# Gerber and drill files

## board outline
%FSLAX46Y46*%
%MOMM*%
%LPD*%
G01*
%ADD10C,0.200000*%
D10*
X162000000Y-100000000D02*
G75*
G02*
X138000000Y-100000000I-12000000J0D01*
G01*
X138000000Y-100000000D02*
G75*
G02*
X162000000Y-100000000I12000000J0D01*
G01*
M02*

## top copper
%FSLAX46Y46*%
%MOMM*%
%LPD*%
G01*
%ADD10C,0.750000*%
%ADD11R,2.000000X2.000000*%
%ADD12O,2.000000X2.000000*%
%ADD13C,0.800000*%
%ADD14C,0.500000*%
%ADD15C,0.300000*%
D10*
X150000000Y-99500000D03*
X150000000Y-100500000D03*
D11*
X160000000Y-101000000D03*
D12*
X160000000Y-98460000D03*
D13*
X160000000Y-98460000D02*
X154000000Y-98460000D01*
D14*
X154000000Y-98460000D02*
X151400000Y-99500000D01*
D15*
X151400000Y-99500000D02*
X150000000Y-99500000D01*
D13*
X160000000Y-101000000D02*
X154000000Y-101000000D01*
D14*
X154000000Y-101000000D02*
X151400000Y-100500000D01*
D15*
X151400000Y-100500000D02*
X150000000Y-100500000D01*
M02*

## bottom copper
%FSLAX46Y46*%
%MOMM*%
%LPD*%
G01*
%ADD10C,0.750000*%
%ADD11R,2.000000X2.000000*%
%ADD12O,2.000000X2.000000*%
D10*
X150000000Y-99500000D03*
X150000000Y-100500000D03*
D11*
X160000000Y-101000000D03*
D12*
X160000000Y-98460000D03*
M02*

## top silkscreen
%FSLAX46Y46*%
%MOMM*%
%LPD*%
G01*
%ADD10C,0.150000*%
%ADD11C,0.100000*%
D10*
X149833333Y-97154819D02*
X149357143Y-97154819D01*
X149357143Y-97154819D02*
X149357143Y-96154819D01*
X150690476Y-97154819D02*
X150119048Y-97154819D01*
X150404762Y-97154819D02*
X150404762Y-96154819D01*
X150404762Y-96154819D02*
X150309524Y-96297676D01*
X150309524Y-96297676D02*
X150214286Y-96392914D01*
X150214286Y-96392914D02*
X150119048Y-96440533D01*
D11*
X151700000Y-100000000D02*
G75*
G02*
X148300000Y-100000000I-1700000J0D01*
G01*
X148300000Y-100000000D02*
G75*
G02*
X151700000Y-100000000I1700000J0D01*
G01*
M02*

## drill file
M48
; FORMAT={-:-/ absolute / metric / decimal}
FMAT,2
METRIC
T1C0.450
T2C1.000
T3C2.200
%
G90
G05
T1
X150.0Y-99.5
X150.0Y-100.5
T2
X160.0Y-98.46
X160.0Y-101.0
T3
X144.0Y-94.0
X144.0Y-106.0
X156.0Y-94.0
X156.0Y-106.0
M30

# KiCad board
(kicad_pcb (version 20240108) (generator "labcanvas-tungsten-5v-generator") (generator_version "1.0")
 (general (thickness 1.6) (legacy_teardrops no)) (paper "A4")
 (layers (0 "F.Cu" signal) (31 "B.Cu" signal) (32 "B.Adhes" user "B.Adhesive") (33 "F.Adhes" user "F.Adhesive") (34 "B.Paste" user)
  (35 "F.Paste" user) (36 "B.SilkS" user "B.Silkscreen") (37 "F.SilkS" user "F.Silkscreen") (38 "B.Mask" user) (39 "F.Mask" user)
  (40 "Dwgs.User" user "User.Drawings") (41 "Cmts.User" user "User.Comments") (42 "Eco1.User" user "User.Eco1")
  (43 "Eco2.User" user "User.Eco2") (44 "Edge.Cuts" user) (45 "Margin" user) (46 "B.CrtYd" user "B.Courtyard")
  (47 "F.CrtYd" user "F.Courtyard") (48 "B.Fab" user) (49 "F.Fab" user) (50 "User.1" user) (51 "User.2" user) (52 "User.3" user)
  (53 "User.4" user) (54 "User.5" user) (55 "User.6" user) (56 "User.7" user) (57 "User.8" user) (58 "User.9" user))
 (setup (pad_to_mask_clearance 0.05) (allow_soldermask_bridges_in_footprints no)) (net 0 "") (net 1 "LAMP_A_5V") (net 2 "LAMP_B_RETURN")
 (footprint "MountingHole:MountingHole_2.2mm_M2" (layer "F.Cu") (at 144 94)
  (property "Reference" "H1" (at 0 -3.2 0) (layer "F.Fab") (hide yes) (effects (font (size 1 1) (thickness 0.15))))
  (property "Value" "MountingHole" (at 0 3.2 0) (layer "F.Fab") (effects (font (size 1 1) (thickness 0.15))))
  (pad "" np_thru_hole circle (at 0 0) (size 2.2 2.2) (drill 2.2) (layers "*.Cu" "*.Mask")))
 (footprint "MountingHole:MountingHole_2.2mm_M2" (layer "F.Cu") (at 156 94)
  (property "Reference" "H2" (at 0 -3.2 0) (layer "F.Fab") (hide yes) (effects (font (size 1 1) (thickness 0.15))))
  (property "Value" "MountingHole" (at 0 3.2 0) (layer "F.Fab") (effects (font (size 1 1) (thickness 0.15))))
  (pad "" np_thru_hole circle (at 0 0) (size 2.2 2.2) (drill 2.2) (layers "*.Cu" "*.Mask")))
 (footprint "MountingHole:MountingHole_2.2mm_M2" (layer "F.Cu") (at 156 106)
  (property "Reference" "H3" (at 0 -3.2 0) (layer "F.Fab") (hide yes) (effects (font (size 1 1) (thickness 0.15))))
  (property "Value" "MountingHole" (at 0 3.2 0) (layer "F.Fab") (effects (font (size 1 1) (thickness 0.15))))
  (pad "" np_thru_hole circle (at 0 0) (size 2.2 2.2) (drill 2.2) (layers "*.Cu" "*.Mask")))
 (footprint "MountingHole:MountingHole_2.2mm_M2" (layer "F.Cu") (at 144 106)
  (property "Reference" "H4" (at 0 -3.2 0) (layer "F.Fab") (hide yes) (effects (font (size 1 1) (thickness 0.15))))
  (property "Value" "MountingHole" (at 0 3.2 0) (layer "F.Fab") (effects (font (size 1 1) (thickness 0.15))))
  (pad "" np_thru_hole circle (at 0 0) (size 2.2 2.2) (drill 2.2) (layers "*.Cu" "*.Mask")))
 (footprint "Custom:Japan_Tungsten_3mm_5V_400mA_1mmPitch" (layer "F.Cu") (at 150 100)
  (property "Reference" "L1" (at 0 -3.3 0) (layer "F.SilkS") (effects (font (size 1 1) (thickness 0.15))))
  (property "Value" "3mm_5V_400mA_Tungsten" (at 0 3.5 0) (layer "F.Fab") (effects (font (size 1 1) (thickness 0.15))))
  (fp_circle (center 0 0) (end 1.7 0) (stroke (width 0.10) (type solid)) (fill none) (layer "F.SilkS"))
  (pad "1" thru_hole circle (at 0 -0.5) (size 0.75 0.75) (drill 0.45) (layers "*.Cu" "*.Mask") (remove_unused_layers no) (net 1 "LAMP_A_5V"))
  (pad "2" thru_hole circle (at 0 0.5) (size 0.75 0.75) (drill 0.45) (layers "*.Cu" "*.Mask") (remove_unused_layers no)
   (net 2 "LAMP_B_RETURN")))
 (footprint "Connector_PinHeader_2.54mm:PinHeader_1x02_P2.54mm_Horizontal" (layer "B.Cu") (at 160 101)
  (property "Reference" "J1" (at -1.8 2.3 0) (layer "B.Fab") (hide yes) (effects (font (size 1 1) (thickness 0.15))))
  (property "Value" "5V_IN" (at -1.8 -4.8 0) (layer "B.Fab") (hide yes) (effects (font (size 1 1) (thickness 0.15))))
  (pad "1" thru_hole rect (at 0 0) (size 2.0 2.0) (drill 1.0) (layers "*.Cu" "*.Mask") (remove_unused_layers no) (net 2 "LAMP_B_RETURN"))
  (pad "2" thru_hole oval (at 0 -2.54) (size 2.0 2.0) (drill 1.0) (layers "*.Cu" "*.Mask") (remove_unused_layers no) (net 1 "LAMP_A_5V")))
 (gr_circle (center 150 100) (end 162 100) (stroke (width 0.2) (type default)) (fill none) (layer "Edge.Cuts"))
 (segment (start 160 98.46) (end 154 98.46) (width 0.8) (layer "F.Cu") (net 1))
 (segment (start 154 98.46) (end 151.4 99.5) (width 0.5) (layer "F.Cu") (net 1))
 (segment (start 151.4 99.5) (end 150 99.5) (width 0.3) (layer "F.Cu") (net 1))
 (segment (start 160 101) (end 154 101) (width 0.8) (layer "F.Cu") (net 2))
 (segment (start 154 101) (end 151.4 100.5) (width 0.5) (layer "F.Cu") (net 2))
 (segment (start 151.4 100.5) (end 150 100.5) (width 0.3) (layer "F.Cu") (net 2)))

